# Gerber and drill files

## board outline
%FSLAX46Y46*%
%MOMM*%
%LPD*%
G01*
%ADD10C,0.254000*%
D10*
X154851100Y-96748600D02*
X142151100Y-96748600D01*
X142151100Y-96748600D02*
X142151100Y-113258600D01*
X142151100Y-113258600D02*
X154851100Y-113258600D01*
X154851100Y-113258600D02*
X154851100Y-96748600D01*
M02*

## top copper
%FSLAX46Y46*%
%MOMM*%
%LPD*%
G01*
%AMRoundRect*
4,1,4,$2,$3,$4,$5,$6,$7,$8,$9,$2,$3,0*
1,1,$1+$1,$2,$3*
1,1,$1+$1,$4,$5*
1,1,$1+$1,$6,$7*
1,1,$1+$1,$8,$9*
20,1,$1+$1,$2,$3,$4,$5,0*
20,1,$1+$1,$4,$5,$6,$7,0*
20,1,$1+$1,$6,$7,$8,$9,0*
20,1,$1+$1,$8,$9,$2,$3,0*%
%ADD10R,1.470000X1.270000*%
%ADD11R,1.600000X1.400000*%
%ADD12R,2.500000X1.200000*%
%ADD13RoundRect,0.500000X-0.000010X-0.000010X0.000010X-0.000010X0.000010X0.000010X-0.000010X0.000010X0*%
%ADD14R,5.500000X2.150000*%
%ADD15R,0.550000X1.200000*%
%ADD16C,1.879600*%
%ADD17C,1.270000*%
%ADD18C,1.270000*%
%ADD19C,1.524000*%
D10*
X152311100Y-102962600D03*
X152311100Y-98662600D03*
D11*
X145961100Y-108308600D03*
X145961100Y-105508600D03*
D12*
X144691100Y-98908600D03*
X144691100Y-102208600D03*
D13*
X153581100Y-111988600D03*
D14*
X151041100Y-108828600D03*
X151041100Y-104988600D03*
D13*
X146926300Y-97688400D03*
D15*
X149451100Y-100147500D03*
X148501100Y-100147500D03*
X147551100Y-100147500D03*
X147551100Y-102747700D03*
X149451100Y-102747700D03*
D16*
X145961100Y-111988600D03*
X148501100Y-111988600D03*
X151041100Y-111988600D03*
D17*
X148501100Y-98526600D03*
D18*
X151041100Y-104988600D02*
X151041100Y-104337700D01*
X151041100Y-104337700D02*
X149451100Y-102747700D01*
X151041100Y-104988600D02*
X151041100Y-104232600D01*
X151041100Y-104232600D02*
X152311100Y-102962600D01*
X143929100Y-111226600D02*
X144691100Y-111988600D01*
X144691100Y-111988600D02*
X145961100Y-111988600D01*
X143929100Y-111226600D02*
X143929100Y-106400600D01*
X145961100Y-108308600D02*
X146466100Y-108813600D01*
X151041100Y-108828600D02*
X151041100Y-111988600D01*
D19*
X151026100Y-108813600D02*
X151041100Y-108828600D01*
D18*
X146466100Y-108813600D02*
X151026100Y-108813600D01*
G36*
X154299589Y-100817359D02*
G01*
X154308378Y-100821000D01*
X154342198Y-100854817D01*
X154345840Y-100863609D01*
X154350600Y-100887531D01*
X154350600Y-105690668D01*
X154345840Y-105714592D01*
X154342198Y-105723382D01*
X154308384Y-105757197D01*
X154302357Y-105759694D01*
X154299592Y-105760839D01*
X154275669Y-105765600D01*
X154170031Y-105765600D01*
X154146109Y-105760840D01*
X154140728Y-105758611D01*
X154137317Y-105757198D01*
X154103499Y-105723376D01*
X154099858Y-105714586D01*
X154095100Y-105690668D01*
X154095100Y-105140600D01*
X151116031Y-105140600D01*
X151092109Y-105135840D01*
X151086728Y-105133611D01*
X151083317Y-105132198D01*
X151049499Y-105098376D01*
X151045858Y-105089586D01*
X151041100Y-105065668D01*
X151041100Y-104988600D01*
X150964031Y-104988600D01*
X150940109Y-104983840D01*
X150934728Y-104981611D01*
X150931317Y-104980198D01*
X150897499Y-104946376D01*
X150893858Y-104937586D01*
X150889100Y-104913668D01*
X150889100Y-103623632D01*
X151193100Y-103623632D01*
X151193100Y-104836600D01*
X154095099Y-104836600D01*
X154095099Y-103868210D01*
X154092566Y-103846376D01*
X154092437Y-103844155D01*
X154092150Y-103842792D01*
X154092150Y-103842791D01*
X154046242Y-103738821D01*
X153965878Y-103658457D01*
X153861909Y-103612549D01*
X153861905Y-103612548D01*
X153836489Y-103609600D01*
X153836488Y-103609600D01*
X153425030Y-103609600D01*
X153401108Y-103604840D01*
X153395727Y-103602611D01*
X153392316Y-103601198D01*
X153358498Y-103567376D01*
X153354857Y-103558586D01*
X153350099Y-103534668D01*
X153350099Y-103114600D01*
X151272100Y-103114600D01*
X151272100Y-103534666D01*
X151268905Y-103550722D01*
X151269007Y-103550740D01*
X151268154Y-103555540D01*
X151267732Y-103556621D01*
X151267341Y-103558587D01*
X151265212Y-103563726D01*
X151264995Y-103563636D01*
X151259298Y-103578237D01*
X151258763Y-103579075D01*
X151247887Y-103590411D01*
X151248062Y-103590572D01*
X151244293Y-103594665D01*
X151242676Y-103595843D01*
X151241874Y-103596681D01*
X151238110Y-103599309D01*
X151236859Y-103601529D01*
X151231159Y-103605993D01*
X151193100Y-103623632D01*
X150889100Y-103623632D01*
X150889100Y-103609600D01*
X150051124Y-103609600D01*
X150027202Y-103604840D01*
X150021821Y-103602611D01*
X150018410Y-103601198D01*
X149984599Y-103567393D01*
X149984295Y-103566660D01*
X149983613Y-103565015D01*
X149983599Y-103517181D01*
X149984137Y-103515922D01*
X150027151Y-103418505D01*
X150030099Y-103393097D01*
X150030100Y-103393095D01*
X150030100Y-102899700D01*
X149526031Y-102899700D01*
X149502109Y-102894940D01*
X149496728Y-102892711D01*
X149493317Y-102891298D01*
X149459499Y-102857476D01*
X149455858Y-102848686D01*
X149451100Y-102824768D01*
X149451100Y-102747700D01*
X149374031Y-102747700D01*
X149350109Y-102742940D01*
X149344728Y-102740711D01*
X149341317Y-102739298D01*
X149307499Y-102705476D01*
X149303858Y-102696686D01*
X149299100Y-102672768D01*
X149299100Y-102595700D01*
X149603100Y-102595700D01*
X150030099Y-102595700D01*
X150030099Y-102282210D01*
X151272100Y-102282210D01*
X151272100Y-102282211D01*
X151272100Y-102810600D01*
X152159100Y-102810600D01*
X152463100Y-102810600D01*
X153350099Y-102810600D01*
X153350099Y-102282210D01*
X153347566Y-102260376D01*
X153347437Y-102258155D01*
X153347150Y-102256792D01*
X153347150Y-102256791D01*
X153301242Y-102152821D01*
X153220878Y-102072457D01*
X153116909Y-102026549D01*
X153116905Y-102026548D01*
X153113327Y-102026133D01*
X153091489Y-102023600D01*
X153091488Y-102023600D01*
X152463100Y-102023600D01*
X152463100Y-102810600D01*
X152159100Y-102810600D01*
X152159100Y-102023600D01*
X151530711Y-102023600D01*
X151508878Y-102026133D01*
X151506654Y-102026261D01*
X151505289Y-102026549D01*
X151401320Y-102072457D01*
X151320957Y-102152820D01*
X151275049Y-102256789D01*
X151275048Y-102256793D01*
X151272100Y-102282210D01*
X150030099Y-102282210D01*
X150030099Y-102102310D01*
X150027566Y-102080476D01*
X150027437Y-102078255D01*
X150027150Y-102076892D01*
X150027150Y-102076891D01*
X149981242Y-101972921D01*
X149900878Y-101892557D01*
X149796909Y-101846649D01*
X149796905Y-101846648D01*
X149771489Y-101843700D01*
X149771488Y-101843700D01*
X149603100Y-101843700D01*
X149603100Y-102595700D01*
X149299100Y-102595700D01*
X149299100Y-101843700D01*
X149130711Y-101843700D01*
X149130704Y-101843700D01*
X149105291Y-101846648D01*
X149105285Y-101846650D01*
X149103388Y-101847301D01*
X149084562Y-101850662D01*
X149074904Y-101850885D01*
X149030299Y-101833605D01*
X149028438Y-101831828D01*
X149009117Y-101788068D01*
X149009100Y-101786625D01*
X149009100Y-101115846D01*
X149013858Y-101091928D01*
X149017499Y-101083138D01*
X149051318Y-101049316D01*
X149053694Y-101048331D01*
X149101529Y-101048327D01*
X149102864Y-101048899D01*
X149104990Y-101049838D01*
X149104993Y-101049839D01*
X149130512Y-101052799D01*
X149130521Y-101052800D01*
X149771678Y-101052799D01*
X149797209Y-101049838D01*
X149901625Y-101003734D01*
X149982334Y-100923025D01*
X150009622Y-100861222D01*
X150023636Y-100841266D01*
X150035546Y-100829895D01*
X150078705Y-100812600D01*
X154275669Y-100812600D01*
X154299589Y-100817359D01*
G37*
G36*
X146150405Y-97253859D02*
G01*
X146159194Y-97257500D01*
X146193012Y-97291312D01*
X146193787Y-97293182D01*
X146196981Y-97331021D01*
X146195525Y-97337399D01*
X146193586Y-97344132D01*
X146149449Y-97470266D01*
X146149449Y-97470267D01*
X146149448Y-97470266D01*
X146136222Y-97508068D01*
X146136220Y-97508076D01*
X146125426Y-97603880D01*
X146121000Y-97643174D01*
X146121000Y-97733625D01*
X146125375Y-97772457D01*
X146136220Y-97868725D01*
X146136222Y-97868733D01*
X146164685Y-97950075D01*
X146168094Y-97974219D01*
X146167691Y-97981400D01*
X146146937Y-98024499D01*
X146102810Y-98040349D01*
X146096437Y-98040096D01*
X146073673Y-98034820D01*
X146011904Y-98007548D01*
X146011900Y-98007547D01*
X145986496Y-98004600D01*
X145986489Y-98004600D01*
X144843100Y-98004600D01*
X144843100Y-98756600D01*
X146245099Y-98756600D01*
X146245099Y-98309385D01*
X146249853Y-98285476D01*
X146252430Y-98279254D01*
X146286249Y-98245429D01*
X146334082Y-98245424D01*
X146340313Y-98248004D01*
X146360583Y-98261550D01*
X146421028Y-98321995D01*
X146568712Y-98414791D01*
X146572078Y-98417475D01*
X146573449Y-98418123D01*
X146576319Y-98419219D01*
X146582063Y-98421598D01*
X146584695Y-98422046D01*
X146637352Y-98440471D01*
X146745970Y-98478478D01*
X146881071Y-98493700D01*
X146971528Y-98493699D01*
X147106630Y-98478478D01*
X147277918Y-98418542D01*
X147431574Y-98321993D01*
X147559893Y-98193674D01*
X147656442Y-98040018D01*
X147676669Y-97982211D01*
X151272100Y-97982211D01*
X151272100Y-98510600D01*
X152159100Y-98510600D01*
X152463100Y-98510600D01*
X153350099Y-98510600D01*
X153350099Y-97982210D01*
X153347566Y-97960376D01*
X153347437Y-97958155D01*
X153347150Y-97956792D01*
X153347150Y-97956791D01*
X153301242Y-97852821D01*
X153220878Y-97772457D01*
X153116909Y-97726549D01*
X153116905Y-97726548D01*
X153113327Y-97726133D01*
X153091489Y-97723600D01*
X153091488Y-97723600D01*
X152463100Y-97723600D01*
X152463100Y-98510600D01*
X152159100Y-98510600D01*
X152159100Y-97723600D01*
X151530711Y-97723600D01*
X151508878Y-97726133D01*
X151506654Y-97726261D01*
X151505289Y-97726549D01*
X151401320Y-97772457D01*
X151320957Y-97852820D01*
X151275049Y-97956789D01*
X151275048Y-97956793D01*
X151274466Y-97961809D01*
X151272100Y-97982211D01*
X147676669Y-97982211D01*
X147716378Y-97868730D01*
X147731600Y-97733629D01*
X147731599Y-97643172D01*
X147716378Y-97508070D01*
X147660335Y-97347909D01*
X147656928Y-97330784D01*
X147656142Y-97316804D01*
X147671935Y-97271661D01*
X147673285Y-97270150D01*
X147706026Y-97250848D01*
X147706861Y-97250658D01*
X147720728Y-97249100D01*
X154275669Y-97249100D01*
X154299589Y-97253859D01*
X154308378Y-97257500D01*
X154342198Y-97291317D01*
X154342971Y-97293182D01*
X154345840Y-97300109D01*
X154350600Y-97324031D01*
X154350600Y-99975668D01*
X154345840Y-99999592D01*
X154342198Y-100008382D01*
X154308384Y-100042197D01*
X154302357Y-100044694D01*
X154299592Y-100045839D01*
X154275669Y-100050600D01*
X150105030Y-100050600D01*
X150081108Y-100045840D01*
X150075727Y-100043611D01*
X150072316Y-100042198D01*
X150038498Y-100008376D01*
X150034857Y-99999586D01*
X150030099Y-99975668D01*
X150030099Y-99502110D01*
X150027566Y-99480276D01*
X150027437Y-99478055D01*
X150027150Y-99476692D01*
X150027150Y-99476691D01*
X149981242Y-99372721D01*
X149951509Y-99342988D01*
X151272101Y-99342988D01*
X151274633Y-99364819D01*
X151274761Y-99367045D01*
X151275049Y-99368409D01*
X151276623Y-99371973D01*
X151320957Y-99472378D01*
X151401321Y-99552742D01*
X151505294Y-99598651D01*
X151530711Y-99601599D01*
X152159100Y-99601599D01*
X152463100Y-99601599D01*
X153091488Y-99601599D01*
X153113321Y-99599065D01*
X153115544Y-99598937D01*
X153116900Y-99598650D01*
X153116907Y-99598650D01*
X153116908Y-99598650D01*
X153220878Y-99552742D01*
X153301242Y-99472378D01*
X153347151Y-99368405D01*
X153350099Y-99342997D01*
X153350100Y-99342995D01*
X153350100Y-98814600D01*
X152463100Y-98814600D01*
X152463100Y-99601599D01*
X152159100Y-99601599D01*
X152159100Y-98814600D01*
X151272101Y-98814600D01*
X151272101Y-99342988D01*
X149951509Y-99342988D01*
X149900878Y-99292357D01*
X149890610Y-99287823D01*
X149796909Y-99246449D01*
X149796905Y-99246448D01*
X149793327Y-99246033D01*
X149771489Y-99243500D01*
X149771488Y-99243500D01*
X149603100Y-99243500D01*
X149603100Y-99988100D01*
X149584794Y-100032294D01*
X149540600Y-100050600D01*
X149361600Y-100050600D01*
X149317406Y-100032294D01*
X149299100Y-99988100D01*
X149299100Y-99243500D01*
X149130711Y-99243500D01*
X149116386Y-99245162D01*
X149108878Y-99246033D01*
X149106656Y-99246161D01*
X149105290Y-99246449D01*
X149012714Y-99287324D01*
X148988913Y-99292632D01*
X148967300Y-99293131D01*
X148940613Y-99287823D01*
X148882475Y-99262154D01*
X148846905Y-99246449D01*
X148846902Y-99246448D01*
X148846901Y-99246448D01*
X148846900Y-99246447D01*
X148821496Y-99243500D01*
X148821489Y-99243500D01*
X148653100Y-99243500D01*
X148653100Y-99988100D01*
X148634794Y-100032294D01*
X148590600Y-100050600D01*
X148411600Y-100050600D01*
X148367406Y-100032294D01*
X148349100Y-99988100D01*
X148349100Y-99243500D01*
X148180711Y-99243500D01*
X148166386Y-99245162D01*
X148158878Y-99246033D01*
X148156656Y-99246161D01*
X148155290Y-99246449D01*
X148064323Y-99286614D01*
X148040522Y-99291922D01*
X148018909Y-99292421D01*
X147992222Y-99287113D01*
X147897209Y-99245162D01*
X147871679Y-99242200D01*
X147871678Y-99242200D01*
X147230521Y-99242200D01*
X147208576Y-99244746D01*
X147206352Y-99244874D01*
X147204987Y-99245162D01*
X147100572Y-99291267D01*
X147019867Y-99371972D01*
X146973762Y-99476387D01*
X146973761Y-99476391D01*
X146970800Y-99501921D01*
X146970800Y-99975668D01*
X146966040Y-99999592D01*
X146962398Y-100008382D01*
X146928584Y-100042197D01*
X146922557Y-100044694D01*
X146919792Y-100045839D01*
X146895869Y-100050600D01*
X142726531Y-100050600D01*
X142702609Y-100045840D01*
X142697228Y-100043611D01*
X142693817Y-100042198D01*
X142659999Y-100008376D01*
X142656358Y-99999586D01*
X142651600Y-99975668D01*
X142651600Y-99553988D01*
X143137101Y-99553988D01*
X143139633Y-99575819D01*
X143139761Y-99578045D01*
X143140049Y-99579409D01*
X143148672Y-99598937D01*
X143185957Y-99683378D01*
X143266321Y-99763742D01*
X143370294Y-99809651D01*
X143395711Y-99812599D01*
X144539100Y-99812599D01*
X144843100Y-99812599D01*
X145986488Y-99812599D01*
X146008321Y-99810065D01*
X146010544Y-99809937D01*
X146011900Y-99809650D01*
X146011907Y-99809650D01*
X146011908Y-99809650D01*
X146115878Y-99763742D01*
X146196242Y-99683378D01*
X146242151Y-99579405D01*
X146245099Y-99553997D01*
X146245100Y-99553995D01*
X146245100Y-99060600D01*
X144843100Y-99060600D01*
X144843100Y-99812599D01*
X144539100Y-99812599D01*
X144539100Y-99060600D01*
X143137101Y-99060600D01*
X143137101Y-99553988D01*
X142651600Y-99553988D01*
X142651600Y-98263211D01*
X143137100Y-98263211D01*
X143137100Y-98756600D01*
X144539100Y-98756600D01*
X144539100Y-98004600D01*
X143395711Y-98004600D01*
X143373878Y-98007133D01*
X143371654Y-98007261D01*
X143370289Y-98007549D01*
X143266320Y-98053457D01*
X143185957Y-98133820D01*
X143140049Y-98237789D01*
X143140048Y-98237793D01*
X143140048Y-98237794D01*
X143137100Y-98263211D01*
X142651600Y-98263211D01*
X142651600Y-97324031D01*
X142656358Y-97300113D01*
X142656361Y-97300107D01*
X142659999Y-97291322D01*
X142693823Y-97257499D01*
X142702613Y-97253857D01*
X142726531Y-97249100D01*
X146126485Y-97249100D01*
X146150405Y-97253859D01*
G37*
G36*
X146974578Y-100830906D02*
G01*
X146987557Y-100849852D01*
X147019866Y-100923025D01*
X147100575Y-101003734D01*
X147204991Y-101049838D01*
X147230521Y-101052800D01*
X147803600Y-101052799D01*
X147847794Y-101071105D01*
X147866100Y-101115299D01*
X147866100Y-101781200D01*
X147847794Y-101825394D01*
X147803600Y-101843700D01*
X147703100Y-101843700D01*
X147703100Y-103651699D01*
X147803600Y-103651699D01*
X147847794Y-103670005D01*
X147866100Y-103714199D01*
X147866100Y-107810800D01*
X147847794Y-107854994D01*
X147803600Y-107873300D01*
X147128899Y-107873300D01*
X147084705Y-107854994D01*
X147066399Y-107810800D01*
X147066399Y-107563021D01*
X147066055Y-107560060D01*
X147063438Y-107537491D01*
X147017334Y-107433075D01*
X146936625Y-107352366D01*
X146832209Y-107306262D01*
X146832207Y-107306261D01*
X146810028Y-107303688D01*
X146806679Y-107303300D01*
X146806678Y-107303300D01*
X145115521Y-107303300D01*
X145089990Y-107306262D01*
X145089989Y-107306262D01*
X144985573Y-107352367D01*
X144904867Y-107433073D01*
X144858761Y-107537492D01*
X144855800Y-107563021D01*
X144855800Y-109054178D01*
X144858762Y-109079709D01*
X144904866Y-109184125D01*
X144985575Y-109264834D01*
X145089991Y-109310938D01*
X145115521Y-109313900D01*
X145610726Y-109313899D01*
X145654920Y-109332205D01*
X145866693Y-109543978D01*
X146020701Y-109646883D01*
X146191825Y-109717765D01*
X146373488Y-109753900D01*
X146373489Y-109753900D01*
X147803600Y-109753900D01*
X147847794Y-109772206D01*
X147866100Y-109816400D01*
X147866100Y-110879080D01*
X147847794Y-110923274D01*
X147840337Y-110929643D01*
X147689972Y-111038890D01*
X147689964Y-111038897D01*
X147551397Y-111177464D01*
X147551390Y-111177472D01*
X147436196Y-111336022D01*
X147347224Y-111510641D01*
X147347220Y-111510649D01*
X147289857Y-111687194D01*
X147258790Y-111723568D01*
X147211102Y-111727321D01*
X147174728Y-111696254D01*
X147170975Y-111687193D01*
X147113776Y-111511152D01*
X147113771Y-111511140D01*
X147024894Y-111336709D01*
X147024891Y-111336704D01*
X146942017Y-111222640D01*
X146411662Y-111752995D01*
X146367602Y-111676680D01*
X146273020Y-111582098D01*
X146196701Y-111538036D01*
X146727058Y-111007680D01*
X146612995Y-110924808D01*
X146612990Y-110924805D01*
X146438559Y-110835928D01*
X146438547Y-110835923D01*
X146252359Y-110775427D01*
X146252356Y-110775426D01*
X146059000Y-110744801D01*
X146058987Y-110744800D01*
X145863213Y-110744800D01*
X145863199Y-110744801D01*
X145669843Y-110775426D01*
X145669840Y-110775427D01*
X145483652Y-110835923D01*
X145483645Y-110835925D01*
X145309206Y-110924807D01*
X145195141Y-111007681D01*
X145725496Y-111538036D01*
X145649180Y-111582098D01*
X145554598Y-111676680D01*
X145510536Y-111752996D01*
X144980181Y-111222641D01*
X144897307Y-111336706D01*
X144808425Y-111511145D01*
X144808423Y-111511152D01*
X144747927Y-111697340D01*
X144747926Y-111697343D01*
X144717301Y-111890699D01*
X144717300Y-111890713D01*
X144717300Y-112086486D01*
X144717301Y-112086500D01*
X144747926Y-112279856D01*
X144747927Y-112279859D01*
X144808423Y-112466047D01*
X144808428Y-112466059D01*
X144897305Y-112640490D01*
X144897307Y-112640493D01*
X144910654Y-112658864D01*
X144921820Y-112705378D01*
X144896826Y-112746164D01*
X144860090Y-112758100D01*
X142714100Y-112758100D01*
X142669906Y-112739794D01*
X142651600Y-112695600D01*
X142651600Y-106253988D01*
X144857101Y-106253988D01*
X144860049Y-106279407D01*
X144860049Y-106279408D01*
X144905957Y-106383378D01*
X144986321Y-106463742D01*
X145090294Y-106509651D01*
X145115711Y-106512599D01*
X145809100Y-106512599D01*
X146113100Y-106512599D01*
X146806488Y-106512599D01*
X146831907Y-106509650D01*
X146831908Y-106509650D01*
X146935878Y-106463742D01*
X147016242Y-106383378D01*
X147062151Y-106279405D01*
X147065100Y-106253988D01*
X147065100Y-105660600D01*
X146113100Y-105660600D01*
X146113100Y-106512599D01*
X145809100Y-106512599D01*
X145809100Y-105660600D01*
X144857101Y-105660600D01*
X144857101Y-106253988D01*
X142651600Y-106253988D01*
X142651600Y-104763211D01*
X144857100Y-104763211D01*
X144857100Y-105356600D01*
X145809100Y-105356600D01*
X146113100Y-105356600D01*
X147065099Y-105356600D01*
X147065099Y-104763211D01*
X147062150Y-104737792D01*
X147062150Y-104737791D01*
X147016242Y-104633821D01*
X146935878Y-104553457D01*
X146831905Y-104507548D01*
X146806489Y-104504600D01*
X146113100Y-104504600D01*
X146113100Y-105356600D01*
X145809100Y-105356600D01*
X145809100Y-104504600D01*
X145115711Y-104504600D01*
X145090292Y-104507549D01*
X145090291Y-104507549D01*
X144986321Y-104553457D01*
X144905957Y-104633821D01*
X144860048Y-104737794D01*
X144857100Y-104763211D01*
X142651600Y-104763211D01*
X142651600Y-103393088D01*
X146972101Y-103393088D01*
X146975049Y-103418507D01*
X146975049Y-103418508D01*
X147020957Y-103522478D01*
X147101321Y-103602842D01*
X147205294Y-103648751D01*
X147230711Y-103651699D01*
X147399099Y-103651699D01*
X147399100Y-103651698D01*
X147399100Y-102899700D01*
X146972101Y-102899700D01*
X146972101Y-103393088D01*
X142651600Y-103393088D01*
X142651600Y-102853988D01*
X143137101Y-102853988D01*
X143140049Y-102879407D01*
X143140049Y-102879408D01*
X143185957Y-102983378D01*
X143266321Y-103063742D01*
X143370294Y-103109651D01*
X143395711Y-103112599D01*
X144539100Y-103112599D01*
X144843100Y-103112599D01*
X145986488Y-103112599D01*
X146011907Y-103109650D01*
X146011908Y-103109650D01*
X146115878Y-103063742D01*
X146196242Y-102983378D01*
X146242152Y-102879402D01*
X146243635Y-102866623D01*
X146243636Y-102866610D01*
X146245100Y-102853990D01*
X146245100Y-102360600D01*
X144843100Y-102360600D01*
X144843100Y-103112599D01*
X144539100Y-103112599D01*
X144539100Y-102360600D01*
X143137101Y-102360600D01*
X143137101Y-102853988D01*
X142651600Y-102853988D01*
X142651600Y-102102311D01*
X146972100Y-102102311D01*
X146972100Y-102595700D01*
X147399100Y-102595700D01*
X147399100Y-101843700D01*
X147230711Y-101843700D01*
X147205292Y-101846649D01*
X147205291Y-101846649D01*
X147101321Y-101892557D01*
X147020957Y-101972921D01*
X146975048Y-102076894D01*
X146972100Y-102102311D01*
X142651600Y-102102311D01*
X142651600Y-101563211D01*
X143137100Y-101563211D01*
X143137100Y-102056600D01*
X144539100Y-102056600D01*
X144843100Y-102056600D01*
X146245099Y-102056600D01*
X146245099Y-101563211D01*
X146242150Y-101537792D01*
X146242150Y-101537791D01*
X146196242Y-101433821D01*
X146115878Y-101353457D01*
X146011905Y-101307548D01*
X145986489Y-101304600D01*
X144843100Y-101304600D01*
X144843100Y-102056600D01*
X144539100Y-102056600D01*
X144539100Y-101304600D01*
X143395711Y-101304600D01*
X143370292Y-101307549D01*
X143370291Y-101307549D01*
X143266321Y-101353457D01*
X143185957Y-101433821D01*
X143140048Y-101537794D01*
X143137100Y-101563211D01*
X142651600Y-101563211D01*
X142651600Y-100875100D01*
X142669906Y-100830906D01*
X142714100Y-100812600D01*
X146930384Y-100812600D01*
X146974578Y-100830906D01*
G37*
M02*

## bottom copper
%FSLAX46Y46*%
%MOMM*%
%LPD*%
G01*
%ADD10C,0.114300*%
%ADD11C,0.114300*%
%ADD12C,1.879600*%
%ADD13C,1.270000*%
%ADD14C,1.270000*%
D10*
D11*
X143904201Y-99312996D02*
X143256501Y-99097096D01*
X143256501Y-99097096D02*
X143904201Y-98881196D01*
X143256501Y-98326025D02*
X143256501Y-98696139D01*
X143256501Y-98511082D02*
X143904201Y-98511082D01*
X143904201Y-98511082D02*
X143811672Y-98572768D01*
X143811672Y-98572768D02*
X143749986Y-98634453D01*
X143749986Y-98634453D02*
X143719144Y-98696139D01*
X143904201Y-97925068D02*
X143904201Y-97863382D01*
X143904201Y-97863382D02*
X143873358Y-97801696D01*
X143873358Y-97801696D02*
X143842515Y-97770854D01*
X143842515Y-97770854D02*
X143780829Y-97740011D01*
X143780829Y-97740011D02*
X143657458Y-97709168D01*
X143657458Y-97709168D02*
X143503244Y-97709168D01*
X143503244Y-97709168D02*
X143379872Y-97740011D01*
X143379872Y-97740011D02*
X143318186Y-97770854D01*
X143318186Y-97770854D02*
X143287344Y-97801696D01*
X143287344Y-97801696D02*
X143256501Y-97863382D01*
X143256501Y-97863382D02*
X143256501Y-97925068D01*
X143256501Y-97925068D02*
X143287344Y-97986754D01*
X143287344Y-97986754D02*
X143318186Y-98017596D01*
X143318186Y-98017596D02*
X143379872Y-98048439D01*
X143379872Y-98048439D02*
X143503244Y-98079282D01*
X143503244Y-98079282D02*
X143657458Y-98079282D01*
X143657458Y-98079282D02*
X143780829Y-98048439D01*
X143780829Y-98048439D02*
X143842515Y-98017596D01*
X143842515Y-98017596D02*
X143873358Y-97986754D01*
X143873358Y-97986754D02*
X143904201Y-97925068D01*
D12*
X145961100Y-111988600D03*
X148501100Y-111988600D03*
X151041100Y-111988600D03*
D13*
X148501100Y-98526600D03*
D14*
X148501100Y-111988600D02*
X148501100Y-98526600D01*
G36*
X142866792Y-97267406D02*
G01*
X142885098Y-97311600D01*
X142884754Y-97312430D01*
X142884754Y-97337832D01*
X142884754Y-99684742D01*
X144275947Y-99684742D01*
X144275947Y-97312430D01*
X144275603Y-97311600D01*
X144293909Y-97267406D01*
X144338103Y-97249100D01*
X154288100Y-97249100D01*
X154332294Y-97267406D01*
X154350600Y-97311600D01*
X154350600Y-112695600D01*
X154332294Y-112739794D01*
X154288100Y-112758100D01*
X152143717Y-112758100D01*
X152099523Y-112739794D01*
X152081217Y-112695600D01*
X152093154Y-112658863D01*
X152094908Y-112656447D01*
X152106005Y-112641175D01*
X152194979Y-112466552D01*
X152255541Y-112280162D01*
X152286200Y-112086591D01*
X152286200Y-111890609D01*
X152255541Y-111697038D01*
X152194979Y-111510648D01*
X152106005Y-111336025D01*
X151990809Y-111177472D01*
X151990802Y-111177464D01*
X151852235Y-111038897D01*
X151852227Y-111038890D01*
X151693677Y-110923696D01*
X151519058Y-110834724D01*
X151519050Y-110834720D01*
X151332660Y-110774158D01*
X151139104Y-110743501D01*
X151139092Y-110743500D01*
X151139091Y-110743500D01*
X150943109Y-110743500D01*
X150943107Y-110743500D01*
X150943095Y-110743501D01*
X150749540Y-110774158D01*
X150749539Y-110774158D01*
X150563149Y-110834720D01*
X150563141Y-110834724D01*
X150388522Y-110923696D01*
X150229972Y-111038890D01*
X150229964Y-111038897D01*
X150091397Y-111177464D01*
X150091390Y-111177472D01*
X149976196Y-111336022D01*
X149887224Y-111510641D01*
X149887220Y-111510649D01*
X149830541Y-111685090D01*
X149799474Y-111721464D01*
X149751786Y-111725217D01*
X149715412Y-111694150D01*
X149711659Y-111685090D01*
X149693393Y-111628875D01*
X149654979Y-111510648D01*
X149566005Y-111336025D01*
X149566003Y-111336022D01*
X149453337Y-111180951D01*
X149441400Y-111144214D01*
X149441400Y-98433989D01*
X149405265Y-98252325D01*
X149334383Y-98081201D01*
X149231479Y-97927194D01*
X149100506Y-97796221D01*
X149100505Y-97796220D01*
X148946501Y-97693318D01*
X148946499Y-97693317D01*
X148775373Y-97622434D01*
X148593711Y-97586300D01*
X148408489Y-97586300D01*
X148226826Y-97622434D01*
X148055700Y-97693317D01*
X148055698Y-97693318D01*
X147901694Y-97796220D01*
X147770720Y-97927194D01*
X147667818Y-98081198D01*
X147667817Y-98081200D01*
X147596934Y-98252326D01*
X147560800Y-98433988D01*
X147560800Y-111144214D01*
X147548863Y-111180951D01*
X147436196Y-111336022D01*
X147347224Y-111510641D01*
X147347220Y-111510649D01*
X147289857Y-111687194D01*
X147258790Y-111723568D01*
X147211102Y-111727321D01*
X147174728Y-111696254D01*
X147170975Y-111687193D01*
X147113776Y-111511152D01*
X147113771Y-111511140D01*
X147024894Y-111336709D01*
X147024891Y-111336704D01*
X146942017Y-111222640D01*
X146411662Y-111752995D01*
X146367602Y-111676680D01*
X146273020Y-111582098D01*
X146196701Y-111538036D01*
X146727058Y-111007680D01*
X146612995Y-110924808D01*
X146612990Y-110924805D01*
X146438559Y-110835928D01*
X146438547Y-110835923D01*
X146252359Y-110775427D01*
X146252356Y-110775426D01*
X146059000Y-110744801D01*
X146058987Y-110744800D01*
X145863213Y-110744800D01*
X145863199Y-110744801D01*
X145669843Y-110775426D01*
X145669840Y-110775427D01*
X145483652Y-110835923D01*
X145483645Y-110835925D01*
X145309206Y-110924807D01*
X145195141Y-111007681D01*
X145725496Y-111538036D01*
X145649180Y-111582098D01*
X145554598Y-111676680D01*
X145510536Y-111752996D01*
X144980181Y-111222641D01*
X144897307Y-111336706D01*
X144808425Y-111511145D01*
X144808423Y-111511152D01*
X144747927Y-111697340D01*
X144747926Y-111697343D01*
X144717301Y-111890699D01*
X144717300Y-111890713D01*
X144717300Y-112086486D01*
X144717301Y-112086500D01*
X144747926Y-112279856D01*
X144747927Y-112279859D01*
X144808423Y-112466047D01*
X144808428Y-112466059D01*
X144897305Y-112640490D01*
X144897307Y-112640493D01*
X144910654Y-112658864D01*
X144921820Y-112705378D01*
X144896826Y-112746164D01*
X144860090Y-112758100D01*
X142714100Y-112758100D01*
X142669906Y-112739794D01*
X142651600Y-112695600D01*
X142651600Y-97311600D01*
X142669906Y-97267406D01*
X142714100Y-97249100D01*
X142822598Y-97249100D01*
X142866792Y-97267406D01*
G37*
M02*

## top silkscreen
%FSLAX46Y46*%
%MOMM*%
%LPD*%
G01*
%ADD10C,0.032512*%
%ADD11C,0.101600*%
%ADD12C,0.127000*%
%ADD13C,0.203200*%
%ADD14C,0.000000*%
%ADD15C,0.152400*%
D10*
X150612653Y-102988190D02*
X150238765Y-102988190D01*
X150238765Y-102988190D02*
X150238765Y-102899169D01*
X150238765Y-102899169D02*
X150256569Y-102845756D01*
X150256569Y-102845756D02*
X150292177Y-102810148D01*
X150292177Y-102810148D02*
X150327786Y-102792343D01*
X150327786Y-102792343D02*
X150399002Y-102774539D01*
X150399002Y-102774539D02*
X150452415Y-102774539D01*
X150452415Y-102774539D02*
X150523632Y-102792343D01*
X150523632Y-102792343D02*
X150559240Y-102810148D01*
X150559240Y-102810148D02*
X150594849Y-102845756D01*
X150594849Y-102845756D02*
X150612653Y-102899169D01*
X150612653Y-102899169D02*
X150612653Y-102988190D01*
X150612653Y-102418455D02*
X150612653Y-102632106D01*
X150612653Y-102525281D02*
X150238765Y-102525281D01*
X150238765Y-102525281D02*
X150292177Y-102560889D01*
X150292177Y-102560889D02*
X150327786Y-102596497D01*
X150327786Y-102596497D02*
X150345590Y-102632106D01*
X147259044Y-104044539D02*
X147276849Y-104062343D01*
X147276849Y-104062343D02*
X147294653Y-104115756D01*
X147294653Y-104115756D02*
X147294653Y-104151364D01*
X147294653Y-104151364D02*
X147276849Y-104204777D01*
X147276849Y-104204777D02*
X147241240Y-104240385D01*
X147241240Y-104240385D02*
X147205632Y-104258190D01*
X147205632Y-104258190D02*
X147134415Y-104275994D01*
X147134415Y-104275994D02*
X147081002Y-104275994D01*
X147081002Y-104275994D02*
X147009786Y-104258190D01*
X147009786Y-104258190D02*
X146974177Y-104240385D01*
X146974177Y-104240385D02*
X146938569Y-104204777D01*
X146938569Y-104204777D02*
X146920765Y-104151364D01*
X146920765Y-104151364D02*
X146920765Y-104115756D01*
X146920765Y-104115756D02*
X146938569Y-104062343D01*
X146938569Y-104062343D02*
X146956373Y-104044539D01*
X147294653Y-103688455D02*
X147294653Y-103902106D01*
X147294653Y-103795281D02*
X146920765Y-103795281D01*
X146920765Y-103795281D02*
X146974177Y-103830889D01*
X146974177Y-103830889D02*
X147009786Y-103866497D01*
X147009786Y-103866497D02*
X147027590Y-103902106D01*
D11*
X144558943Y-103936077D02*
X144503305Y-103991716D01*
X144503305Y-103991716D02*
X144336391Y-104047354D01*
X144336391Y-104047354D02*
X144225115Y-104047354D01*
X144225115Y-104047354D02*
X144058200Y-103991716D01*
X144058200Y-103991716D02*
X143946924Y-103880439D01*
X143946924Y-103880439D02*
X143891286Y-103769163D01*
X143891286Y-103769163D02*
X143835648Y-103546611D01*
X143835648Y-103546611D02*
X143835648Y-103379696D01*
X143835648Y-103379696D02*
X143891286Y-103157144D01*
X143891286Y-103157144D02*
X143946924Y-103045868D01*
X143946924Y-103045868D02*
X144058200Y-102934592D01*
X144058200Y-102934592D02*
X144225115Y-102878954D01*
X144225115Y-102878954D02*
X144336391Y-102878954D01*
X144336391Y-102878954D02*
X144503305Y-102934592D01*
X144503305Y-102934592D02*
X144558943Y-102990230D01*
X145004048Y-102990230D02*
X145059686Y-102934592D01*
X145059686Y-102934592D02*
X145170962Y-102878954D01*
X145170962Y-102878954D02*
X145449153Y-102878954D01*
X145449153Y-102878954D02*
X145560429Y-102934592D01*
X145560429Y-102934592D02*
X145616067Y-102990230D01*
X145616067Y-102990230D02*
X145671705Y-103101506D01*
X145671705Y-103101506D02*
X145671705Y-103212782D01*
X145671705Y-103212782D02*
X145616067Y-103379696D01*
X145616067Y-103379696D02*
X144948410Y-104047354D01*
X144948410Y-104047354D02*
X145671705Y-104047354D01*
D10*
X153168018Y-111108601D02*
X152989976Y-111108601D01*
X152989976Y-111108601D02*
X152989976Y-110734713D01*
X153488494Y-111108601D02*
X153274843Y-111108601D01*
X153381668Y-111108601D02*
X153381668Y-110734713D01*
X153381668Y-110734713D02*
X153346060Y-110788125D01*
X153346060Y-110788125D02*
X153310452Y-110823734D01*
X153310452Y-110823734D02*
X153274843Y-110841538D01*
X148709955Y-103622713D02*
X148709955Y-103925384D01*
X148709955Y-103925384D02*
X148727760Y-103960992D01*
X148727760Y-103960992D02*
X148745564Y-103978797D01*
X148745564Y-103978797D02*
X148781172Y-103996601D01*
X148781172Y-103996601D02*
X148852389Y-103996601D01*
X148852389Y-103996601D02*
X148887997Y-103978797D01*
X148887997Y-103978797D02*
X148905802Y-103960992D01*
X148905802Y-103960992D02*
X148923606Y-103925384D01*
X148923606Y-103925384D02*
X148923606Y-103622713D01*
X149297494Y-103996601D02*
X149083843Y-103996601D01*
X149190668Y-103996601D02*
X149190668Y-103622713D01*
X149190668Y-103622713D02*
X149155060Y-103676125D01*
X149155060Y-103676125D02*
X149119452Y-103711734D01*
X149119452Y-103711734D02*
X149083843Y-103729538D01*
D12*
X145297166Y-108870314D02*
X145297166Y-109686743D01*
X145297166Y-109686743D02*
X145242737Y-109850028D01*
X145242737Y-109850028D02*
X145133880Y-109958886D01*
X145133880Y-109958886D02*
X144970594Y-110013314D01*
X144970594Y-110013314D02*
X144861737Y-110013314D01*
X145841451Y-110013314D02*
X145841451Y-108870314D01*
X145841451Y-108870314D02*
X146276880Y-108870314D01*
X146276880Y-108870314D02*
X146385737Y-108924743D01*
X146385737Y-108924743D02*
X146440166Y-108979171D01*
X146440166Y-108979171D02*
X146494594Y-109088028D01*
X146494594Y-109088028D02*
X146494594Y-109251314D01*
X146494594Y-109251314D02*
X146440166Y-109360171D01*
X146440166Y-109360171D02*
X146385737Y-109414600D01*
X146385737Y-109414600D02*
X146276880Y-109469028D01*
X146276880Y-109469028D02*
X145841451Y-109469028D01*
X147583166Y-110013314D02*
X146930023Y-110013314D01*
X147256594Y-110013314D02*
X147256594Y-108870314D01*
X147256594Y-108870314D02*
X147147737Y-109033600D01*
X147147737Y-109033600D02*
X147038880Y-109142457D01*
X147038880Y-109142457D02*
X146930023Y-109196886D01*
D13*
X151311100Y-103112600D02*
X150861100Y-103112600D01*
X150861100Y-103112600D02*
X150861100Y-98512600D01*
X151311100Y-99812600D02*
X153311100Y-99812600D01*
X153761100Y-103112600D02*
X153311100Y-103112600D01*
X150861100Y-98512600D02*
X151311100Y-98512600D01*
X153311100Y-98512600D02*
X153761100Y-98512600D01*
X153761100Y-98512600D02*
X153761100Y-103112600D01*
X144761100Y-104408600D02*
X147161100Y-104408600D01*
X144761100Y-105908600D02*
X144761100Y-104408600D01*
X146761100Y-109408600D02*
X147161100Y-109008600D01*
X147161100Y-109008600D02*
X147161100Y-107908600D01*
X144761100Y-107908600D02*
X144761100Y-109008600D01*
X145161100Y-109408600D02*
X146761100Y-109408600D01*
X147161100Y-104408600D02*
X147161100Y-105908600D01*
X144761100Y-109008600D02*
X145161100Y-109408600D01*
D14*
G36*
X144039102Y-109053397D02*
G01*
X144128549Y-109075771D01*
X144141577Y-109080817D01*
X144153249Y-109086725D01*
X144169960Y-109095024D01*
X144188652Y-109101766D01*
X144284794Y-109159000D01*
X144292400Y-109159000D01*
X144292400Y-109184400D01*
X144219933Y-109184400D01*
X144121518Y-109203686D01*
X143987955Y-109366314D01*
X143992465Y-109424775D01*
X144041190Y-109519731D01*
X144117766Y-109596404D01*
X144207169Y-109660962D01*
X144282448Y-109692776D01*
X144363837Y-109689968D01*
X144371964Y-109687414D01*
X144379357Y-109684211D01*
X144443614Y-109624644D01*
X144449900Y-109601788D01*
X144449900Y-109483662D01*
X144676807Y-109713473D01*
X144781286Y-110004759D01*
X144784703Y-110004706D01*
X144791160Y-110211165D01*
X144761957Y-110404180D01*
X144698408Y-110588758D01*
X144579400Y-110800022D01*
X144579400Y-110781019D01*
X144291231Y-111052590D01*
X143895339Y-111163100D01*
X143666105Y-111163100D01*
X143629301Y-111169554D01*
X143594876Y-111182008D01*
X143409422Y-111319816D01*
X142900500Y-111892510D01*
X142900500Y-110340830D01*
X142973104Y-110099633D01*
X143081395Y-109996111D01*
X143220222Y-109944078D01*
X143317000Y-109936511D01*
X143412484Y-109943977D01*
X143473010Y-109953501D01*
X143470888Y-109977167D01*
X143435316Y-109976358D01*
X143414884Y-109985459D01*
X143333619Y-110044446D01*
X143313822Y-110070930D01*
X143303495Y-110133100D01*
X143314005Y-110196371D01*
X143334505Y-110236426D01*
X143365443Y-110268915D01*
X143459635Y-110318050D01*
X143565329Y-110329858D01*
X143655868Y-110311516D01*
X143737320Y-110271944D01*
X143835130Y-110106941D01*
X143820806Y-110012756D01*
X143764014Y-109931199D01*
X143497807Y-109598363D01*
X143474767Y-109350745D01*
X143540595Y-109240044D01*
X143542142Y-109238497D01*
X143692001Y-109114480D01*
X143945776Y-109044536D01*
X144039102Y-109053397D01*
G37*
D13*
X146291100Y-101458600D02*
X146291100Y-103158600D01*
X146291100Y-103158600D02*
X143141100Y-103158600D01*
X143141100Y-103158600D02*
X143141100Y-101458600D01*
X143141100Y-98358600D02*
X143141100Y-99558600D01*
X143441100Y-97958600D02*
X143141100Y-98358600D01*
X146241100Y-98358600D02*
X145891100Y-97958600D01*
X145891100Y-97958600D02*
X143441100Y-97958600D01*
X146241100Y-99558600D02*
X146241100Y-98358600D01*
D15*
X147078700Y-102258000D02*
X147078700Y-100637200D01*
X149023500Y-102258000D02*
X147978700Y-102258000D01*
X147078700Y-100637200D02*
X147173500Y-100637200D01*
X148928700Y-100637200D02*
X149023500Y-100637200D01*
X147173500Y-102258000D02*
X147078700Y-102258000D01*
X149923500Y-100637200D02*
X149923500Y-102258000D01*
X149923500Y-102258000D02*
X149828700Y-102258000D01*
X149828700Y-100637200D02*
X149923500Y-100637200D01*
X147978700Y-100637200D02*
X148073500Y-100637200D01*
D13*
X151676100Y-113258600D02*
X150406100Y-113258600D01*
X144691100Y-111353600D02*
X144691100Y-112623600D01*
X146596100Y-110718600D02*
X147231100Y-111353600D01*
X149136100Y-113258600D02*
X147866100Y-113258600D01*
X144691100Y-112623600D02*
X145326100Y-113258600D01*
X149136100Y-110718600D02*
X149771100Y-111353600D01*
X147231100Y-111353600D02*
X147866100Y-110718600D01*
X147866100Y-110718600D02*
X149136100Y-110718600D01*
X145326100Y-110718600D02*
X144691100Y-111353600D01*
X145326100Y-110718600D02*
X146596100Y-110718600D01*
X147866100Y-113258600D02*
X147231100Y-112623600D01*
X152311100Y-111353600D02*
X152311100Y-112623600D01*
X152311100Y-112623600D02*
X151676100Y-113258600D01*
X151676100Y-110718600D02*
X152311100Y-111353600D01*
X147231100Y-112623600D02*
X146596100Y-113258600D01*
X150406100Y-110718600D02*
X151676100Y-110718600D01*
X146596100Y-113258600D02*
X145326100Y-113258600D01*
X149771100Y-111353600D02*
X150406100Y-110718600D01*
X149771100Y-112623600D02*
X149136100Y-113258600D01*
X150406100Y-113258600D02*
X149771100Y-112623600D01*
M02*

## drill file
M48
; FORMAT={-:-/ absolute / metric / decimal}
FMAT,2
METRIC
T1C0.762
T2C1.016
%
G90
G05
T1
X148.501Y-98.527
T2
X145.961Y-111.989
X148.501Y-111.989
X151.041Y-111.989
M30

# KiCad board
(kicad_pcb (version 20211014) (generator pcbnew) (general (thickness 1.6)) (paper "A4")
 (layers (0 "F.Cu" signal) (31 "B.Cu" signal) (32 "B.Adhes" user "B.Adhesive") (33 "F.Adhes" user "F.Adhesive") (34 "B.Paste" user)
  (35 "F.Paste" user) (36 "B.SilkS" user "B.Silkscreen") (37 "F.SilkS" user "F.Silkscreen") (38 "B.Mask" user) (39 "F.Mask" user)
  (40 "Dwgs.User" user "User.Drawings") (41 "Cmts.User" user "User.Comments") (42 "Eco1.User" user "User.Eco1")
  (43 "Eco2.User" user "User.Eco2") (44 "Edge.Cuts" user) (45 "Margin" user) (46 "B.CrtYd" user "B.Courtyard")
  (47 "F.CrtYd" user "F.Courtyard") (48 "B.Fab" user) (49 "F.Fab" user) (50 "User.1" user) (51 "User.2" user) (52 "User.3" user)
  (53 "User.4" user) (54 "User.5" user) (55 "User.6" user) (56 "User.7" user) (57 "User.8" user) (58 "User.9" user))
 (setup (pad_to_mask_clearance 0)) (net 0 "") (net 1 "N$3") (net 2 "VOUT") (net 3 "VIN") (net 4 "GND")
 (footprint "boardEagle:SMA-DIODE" (layer "F.Cu") (at 152.3111 100.8126 90)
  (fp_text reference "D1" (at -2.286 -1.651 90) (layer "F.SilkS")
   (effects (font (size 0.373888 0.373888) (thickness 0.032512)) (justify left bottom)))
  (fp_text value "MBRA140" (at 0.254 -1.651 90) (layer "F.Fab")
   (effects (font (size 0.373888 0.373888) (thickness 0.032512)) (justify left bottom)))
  (fp_line (start -2.3 -1) (end -2.3 -1.45) (layer "F.SilkS") (width 0.2032))
  (fp_line (start -2.3 -1.45) (end 2.3 -1.45) (layer "F.SilkS") (width 0.2032))
  (fp_line (start 1 -1) (end 1 1) (layer "F.SilkS") (width 0.2032))
  (fp_line (start -2.3 1.45) (end -2.3 1) (layer "F.SilkS") (width 0.2032))
  (fp_line (start 2.3 -1.45) (end 2.3 -1) (layer "F.SilkS") (width 0.2032))
  (fp_line (start 2.3 1) (end 2.3 1.45) (layer "F.SilkS") (width 0.2032))
  (fp_line (start 2.3 1.45) (end -2.3 1.45) (layer "F.SilkS") (width 0.2032))
  (pad "A" smd rect (at -2.15 0 270) (size 1.27 1.47) (layers "F.Cu" "F.Paste" "F.Mask") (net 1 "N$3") (solder_mask_margin 0.1016))
  (pad "C" smd rect (at 2.15 0 90) (size 1.27 1.47) (layers "F.Cu" "F.Paste" "F.Mask") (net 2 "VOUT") (solder_mask_margin 0.1016)))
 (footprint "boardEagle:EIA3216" (layer "F.Cu") (at 145.9611 106.9086 -90)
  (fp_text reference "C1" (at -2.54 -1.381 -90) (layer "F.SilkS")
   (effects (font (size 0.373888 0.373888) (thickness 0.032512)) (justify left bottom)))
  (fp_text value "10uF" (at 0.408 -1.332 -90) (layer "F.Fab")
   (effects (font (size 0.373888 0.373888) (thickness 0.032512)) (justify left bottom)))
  (fp_line (start -2.5 1.2) (end -2.5 -1.2) (layer "F.SilkS") (width 0.2032))
  (fp_line (start -1 1.2) (end -2.5 1.2) (layer "F.SilkS") (width 0.2032))
  (fp_line (start 2.5 -0.8) (end 2.1 -1.2) (layer "F.SilkS") (width 0.2032))
  (fp_line (start 2.1 -1.2) (end 1 -1.2) (layer "F.SilkS") (width 0.2032))
  (fp_line (start 1 1.2) (end 2.1 1.2) (layer "F.SilkS") (width 0.2032))
  (fp_line (start 2.5 0.8) (end 2.5 -0.8) (layer "F.SilkS") (width 0.2032))
  (fp_line (start -2.5 -1.2) (end -1 -1.2) (layer "F.SilkS") (width 0.2032))
  (fp_line (start 2.1 1.2) (end 2.5 0.8) (layer "F.SilkS") (width 0.2032))
  (pad "A" smd rect (at 1.4 0) (size 1.6 1.4) (layers "F.Cu" "F.Paste" "F.Mask") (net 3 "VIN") (solder_mask_margin 0.1016))
  (pad "C" smd rect (at -1.4 0) (size 1.6 1.4) (layers "F.Cu" "F.Paste" "F.Mask") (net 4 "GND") (solder_mask_margin 0.1016)))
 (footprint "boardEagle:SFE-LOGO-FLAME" (layer "F.Cu") (at 142.9131 111.8616)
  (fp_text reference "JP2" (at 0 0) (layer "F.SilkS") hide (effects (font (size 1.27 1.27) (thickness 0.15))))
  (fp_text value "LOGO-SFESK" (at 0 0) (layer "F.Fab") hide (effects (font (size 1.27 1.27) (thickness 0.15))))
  (fp_poly
   (pts (xy 1.126002 -2.808203) (xy 1.215449 -2.785829) (xy 1.228477 -2.780783) (xy 1.240149 -2.774875) (xy 1.25686 -2.766576)
    (xy 1.275552 -2.759834) (xy 1.371694 -2.7026) (xy 1.3793 -2.7026) (xy 1.3793 -2.6772) (xy 1.306833 -2.6772) (xy 1.208418 -2.657914)
    (xy 1.074855 -2.495286) (xy 1.079365 -2.436825) (xy 1.12809 -2.341869) (xy 1.204666 -2.265196) (xy 1.294069 -2.200638)
    (xy 1.369348 -2.168824) (xy 1.450737 -2.171632) (xy 1.458864 -2.174186) (xy 1.466257 -2.177389) (xy 1.530514 -2.236956)
    (xy 1.5368 -2.259812) (xy 1.5368 -2.377938) (xy 1.763707 -2.148127) (xy 1.868186 -1.856841) (xy 1.871603 -1.856894)
    (xy 1.87806 -1.650435) (xy 1.848857 -1.45742) (xy 1.785308 -1.272842) (xy 1.6663 -1.061578) (xy 1.6663 -1.080581) (xy 1.378131 -0.80901)
    (xy 0.982239 -0.6985) (xy 0.753005 -0.6985) (xy 0.716201 -0.692046) (xy 0.681776 -0.679592) (xy 0.496322 -0.541784) (xy -0.0126 0.03091)
    (xy -0.0126 -1.52077) (xy 0.060004 -1.761967) (xy 0.168295 -1.865489) (xy 0.307122 -1.917522) (xy 0.4039 -1.925089)
    (xy 0.499384 -1.917623) (xy 0.55991 -1.908099) (xy 0.557788 -1.884433) (xy 0.522216 -1.885242) (xy 0.501784 -1.876141)
    (xy 0.420519 -1.817154) (xy 0.400722 -1.79067) (xy 0.390395 -1.7285) (xy 0.400905 -1.665229) (xy 0.421405 -1.625174)
    (xy 0.452343 -1.592685) (xy 0.546535 -1.54355) (xy 0.652229 -1.531742) (xy 0.742768 -1.550084) (xy 0.82422 -1.589656)
    (xy 0.92203 -1.754659) (xy 0.907706 -1.848844) (xy 0.850914 -1.930401) (xy 0.584707 -2.263237) (xy 0.561667 -2.510855)
    (xy 0.627495 -2.621556) (xy 0.629042 -2.623103) (xy 0.778901 -2.74712) (xy 1.032676 -2.817064))
   (layer "F.SilkS") (width 0) (fill solid)))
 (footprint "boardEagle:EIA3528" (layer "F.Cu") (at 144.6911 100.5586 90)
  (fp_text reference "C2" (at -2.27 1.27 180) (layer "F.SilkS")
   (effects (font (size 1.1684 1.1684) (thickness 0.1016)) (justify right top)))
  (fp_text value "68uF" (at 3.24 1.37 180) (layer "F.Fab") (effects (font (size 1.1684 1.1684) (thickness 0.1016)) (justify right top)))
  (fp_line (start -0.9 1.6) (end -2.6 1.6) (layer "F.SilkS") (width 0.2032))
  (fp_line (start -2.6 1.6) (end -2.6 -1.55) (layer "F.SilkS") (width 0.2032))
  (fp_line (start -2.6 -1.55) (end -0.9 -1.55) (layer "F.SilkS") (width 0.2032))
  (fp_line (start 2.2 -1.55) (end 1 -1.55) (layer "F.SilkS") (width 0.2032))
  (fp_line (start 2.6 -1.25) (end 2.2 -1.55) (layer "F.SilkS") (width 0.2032))
  (fp_line (start 2.2 1.55) (end 2.6 1.2) (layer "F.SilkS") (width 0.2032))
  (fp_line (start 2.6 1.2) (end 2.6 -1.25) (layer "F.SilkS") (width 0.2032))
  (fp_line (start 1 1.55) (end 2.2 1.55) (layer "F.SilkS") (width 0.2032))
  (pad "A" smd rect (at 1.65 0 180) (size 2.5 1.2) (layers "F.Cu" "F.Paste" "F.Mask") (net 2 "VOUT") (solder_mask_margin 0.1016))
  (pad "C" smd rect (at -1.65 0 180) (size 2.5 1.2) (layers "F.Cu" "F.Paste" "F.Mask") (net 4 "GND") (solder_mask_margin 0.1016)))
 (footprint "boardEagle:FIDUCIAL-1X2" (layer "F.Cu") (at 153.5811 111.9886)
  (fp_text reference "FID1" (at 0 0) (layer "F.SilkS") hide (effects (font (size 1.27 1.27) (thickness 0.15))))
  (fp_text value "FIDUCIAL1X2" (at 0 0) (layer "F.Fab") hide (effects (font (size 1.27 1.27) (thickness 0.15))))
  (pad "1" smd roundrect (at 0 0) (size 1 1) (layers "F.Cu" "F.Mask") (roundrect_rratio 0.5) (solder_mask_margin 0.1016)))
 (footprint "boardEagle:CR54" (layer "F.Cu") (at 151.0411 106.9086 180)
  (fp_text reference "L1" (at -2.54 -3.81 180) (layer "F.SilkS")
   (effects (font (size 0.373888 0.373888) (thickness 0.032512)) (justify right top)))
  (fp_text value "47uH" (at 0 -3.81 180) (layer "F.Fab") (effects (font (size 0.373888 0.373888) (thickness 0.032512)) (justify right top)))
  (pad "P$1" smd rect (at 0 -1.92 180) (size 5.5 2.15) (layers "F.Cu" "F.Paste" "F.Mask") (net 3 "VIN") (solder_mask_margin 0.1016))
  (pad "P$2" smd rect (at 0 1.92 180) (size 5.5 2.15) (layers "F.Cu" "F.Paste" "F.Mask") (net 1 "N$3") (solder_mask_margin 0.1016)))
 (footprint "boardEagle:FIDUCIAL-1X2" (layer "F.Cu") (at 146.9263 97.6884)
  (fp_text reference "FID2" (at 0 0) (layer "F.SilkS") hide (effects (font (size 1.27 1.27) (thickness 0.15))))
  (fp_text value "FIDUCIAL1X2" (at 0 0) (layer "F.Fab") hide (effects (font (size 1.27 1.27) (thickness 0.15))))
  (pad "1" smd roundrect (at 0 0) (size 1 1) (layers "F.Cu" "F.Mask") (roundrect_rratio 0.5) (solder_mask_margin 0.1016)))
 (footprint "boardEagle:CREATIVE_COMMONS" (layer "F.Cu") (at 43.871622 113.2586)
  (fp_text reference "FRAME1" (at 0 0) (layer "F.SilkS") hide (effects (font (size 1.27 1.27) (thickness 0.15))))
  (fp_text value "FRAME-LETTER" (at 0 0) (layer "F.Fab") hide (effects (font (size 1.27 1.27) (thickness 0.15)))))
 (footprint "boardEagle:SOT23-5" (layer "F.Cu") (at 148.5011 101.4476 180)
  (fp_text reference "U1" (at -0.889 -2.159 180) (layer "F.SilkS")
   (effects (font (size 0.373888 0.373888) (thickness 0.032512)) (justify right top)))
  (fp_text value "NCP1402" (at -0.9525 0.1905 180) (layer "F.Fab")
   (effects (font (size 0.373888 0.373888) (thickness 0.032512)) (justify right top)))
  (fp_line (start 1.4224 -0.8104) (end 1.4224 0.8104) (layer "F.SilkS") (width 0.1524))
  (fp_line (start -0.5224 -0.8104) (end 0.5224 -0.8104) (layer "F.SilkS") (width 0.1524))
  (fp_line (start 1.4224 0.8104) (end 1.3276 0.8104) (layer "F.SilkS") (width 0.1524))
  (fp_line (start -0.4276 0.8104) (end -0.5224 0.8104) (layer "F.SilkS") (width 0.1524))
  (fp_line (start 1.3276 -0.8104) (end 1.4224 -0.8104) (layer "F.SilkS") (width 0.1524))
  (fp_line (start -1.4224 0.8104) (end -1.4224 -0.8104) (layer "F.SilkS") (width 0.1524))
  (fp_line (start -1.4224 -0.8104) (end -1.3276 -0.8104) (layer "F.SilkS") (width 0.1524))
  (fp_line (start -1.3276 0.8104) (end -1.4224 0.8104) (layer "F.SilkS") (width 0.1524))
  (fp_line (start 0.5224 0.8104) (end 0.4276 0.8104) (layer "F.SilkS") (width 0.1524))
  (pad "1" smd rect (at -0.95 1.3001 180) (size 0.55 1.2) (layers "F.Cu" "F.Paste" "F.Mask") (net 2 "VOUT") (solder_mask_margin 0.1016))
  (pad "2" smd rect (at 0 1.3001 180) (size 0.55 1.2) (layers "F.Cu" "F.Paste" "F.Mask") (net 2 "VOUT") (solder_mask_margin 0.1016))
  (pad "3" smd rect (at 0.95 1.3001 180) (size 0.55 1.2) (layers "F.Cu" "F.Paste" "F.Mask") (solder_mask_margin 0.1016))
  (pad "4" smd rect (at 0.95 -1.3001 180) (size 0.55 1.2) (layers "F.Cu" "F.Paste" "F.Mask") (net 4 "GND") (solder_mask_margin 0.1016))
  (pad "5" smd rect (at -0.95 -1.3001 180) (size 0.55 1.2) (layers "F.Cu" "F.Paste" "F.Mask") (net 1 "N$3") (solder_mask_margin 0.1016)))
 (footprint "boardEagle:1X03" (layer "F.Cu") (at 145.9611 111.9886)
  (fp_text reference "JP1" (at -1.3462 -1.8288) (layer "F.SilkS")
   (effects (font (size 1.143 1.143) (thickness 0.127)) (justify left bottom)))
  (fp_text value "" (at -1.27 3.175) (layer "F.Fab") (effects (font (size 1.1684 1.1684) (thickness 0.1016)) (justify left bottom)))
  (fp_line (start 5.715 1.27) (end 4.445 1.27) (layer "F.SilkS") (width 0.2032))
  (fp_line (start -1.27 -0.635) (end -1.27 0.635) (layer "F.SilkS") (width 0.2032))
  (fp_line (start 0.635 -1.27) (end 1.27 -0.635) (layer "F.SilkS") (width 0.2032))
  (fp_line (start 3.175 1.27) (end 1.905 1.27) (layer "F.SilkS") (width 0.2032))
  (fp_line (start -1.27 0.635) (end -0.635 1.27) (layer "F.SilkS") (width 0.2032))
  (fp_line (start 3.175 -1.27) (end 3.81 -0.635) (layer "F.SilkS") (width 0.2032))
  (fp_line (start 1.27 -0.635) (end 1.905 -1.27) (layer "F.SilkS") (width 0.2032))
  (fp_line (start 1.905 -1.27) (end 3.175 -1.27) (layer "F.SilkS") (width 0.2032))
  (fp_line (start -0.635 -1.27) (end -1.27 -0.635) (layer "F.SilkS") (width 0.2032))
  (fp_line (start -0.635 -1.27) (end 0.635 -1.27) (layer "F.SilkS") (width 0.2032))
  (fp_line (start 1.905 1.27) (end 1.27 0.635) (layer "F.SilkS") (width 0.2032))
  (fp_line (start 6.35 -0.635) (end 6.35 0.635) (layer "F.SilkS") (width 0.2032))
  (fp_line (start 6.35 0.635) (end 5.715 1.27) (layer "F.SilkS") (width 0.2032))
  (fp_line (start 5.715 -1.27) (end 6.35 -0.635) (layer "F.SilkS") (width 0.2032))
  (fp_line (start 1.27 0.635) (end 0.635 1.27) (layer "F.SilkS") (width 0.2032))
  (fp_line (start 4.445 -1.27) (end 5.715 -1.27) (layer "F.SilkS") (width 0.2032))
  (fp_line (start 0.635 1.27) (end -0.635 1.27) (layer "F.SilkS") (width 0.2032))
  (fp_line (start 3.81 -0.635) (end 4.445 -1.27) (layer "F.SilkS") (width 0.2032))
  (fp_line (start 3.81 0.635) (end 3.175 1.27) (layer "F.SilkS") (width 0.2032))
  (fp_line (start 4.445 1.27) (end 3.81 0.635) (layer "F.SilkS") (width 0.2032))
  (pad "1" thru_hole circle (at 0 0 90) (size 1.8796 1.8796) (drill 1.016) (layers *.Cu *.Mask) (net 4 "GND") (solder_mask_margin 0.1016))
  (pad "2" thru_hole circle (at 2.54 0 90) (size 1.8796 1.8796) (drill 1.016) (layers *.Cu *.Mask) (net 2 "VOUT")
   (solder_mask_margin 0.1016))
  (pad "3" thru_hole circle (at 5.08 0 90) (size 1.8796 1.8796) (drill 1.016) (layers *.Cu *.Mask) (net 3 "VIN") (solder_mask_margin 0.1016)))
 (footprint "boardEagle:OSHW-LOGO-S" (layer "B.Cu") (at 152.3111 99.2886 90)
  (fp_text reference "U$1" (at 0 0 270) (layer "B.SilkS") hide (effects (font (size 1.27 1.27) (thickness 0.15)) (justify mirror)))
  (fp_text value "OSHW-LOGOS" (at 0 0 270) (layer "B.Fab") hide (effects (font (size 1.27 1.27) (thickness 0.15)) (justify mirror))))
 (gr_line (start 154.8511 96.7486) (end 142.1511 96.7486) (layer "Edge.Cuts") (width 0.254))
 (gr_line (start 142.1511 96.7486) (end 142.1511 113.2586) (layer "Edge.Cuts") (width 0.254))
 (gr_line (start 142.1511 113.2586) (end 154.8511 113.2586) (layer "Edge.Cuts") (width 0.254))
 (gr_line (start 154.8511 113.2586) (end 154.8511 96.7486) (layer "Edge.Cuts") (width 0.254))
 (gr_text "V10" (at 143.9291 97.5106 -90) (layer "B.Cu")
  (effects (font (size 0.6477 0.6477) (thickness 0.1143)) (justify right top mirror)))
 (segment (start 151.0411 104.9886) (end 151.0411 104.3377) (width 1.27) (layer "F.Cu") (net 1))
 (segment (start 151.0411 104.3377) (end 149.4511 102.7477) (width 1.27) (layer "F.Cu") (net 1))
 (segment (start 151.0411 104.9886) (end 151.0411 104.2326) (width 1.27) (layer "F.Cu") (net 1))
 (segment (start 151.0411 104.2326) (end 152.3111 102.9626) (width 1.27) (layer "F.Cu") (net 1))
 (via (at 148.5011 98.5266) (size 1.27) (drill 0.762) (layers "F.Cu" "B.Cu") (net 2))
 (segment (start 148.5011 111.9886) (end 148.5011 98.5266) (width 1.27) (layer "B.Cu") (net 2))
 (segment (start 143.9291 111.2266) (end 144.6911 111.9886) (width 1.27) (layer "F.Cu") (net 4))
 (segment (start 144.6911 111.9886) (end 145.9611 111.9886) (width 1.27) (layer "F.Cu") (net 4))
 (segment (start 143.9291 111.2266) (end 143.9291 106.4006) (width 1.27) (layer "F.Cu") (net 4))
 (segment (start 145.9611 108.3086) (end 146.4661 108.8136) (width 1.27) (layer "F.Cu") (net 3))
 (segment (start 151.0411 108.8286) (end 151.0411 111.9886) (width 1.27) (layer "F.Cu") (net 3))
 (segment (start 151.0261 108.8136) (end 151.0411 108.8286) (width 1.524) (layer "F.Cu") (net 3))
 (segment (start 146.4661 108.8136) (end 151.0261 108.8136) (width 1.27) (layer "F.Cu") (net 3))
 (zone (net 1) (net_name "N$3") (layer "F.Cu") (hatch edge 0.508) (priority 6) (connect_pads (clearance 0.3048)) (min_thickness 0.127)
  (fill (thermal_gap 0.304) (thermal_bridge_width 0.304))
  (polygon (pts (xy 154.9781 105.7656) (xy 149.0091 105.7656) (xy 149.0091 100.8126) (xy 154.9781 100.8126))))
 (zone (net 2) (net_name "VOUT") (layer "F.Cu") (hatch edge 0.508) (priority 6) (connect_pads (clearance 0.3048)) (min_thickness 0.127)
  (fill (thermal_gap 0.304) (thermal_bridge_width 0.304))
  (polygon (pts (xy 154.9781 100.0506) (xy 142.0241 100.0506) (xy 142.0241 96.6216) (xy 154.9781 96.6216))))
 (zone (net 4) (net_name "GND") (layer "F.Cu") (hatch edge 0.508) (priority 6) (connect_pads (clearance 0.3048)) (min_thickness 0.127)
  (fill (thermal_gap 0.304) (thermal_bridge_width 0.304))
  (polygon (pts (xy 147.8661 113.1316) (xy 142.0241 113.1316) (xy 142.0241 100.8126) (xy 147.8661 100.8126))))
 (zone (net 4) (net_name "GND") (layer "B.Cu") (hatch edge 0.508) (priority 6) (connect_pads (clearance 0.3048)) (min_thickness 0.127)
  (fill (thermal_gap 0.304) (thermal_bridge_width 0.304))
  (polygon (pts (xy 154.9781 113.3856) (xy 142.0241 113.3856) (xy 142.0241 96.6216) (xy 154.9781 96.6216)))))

